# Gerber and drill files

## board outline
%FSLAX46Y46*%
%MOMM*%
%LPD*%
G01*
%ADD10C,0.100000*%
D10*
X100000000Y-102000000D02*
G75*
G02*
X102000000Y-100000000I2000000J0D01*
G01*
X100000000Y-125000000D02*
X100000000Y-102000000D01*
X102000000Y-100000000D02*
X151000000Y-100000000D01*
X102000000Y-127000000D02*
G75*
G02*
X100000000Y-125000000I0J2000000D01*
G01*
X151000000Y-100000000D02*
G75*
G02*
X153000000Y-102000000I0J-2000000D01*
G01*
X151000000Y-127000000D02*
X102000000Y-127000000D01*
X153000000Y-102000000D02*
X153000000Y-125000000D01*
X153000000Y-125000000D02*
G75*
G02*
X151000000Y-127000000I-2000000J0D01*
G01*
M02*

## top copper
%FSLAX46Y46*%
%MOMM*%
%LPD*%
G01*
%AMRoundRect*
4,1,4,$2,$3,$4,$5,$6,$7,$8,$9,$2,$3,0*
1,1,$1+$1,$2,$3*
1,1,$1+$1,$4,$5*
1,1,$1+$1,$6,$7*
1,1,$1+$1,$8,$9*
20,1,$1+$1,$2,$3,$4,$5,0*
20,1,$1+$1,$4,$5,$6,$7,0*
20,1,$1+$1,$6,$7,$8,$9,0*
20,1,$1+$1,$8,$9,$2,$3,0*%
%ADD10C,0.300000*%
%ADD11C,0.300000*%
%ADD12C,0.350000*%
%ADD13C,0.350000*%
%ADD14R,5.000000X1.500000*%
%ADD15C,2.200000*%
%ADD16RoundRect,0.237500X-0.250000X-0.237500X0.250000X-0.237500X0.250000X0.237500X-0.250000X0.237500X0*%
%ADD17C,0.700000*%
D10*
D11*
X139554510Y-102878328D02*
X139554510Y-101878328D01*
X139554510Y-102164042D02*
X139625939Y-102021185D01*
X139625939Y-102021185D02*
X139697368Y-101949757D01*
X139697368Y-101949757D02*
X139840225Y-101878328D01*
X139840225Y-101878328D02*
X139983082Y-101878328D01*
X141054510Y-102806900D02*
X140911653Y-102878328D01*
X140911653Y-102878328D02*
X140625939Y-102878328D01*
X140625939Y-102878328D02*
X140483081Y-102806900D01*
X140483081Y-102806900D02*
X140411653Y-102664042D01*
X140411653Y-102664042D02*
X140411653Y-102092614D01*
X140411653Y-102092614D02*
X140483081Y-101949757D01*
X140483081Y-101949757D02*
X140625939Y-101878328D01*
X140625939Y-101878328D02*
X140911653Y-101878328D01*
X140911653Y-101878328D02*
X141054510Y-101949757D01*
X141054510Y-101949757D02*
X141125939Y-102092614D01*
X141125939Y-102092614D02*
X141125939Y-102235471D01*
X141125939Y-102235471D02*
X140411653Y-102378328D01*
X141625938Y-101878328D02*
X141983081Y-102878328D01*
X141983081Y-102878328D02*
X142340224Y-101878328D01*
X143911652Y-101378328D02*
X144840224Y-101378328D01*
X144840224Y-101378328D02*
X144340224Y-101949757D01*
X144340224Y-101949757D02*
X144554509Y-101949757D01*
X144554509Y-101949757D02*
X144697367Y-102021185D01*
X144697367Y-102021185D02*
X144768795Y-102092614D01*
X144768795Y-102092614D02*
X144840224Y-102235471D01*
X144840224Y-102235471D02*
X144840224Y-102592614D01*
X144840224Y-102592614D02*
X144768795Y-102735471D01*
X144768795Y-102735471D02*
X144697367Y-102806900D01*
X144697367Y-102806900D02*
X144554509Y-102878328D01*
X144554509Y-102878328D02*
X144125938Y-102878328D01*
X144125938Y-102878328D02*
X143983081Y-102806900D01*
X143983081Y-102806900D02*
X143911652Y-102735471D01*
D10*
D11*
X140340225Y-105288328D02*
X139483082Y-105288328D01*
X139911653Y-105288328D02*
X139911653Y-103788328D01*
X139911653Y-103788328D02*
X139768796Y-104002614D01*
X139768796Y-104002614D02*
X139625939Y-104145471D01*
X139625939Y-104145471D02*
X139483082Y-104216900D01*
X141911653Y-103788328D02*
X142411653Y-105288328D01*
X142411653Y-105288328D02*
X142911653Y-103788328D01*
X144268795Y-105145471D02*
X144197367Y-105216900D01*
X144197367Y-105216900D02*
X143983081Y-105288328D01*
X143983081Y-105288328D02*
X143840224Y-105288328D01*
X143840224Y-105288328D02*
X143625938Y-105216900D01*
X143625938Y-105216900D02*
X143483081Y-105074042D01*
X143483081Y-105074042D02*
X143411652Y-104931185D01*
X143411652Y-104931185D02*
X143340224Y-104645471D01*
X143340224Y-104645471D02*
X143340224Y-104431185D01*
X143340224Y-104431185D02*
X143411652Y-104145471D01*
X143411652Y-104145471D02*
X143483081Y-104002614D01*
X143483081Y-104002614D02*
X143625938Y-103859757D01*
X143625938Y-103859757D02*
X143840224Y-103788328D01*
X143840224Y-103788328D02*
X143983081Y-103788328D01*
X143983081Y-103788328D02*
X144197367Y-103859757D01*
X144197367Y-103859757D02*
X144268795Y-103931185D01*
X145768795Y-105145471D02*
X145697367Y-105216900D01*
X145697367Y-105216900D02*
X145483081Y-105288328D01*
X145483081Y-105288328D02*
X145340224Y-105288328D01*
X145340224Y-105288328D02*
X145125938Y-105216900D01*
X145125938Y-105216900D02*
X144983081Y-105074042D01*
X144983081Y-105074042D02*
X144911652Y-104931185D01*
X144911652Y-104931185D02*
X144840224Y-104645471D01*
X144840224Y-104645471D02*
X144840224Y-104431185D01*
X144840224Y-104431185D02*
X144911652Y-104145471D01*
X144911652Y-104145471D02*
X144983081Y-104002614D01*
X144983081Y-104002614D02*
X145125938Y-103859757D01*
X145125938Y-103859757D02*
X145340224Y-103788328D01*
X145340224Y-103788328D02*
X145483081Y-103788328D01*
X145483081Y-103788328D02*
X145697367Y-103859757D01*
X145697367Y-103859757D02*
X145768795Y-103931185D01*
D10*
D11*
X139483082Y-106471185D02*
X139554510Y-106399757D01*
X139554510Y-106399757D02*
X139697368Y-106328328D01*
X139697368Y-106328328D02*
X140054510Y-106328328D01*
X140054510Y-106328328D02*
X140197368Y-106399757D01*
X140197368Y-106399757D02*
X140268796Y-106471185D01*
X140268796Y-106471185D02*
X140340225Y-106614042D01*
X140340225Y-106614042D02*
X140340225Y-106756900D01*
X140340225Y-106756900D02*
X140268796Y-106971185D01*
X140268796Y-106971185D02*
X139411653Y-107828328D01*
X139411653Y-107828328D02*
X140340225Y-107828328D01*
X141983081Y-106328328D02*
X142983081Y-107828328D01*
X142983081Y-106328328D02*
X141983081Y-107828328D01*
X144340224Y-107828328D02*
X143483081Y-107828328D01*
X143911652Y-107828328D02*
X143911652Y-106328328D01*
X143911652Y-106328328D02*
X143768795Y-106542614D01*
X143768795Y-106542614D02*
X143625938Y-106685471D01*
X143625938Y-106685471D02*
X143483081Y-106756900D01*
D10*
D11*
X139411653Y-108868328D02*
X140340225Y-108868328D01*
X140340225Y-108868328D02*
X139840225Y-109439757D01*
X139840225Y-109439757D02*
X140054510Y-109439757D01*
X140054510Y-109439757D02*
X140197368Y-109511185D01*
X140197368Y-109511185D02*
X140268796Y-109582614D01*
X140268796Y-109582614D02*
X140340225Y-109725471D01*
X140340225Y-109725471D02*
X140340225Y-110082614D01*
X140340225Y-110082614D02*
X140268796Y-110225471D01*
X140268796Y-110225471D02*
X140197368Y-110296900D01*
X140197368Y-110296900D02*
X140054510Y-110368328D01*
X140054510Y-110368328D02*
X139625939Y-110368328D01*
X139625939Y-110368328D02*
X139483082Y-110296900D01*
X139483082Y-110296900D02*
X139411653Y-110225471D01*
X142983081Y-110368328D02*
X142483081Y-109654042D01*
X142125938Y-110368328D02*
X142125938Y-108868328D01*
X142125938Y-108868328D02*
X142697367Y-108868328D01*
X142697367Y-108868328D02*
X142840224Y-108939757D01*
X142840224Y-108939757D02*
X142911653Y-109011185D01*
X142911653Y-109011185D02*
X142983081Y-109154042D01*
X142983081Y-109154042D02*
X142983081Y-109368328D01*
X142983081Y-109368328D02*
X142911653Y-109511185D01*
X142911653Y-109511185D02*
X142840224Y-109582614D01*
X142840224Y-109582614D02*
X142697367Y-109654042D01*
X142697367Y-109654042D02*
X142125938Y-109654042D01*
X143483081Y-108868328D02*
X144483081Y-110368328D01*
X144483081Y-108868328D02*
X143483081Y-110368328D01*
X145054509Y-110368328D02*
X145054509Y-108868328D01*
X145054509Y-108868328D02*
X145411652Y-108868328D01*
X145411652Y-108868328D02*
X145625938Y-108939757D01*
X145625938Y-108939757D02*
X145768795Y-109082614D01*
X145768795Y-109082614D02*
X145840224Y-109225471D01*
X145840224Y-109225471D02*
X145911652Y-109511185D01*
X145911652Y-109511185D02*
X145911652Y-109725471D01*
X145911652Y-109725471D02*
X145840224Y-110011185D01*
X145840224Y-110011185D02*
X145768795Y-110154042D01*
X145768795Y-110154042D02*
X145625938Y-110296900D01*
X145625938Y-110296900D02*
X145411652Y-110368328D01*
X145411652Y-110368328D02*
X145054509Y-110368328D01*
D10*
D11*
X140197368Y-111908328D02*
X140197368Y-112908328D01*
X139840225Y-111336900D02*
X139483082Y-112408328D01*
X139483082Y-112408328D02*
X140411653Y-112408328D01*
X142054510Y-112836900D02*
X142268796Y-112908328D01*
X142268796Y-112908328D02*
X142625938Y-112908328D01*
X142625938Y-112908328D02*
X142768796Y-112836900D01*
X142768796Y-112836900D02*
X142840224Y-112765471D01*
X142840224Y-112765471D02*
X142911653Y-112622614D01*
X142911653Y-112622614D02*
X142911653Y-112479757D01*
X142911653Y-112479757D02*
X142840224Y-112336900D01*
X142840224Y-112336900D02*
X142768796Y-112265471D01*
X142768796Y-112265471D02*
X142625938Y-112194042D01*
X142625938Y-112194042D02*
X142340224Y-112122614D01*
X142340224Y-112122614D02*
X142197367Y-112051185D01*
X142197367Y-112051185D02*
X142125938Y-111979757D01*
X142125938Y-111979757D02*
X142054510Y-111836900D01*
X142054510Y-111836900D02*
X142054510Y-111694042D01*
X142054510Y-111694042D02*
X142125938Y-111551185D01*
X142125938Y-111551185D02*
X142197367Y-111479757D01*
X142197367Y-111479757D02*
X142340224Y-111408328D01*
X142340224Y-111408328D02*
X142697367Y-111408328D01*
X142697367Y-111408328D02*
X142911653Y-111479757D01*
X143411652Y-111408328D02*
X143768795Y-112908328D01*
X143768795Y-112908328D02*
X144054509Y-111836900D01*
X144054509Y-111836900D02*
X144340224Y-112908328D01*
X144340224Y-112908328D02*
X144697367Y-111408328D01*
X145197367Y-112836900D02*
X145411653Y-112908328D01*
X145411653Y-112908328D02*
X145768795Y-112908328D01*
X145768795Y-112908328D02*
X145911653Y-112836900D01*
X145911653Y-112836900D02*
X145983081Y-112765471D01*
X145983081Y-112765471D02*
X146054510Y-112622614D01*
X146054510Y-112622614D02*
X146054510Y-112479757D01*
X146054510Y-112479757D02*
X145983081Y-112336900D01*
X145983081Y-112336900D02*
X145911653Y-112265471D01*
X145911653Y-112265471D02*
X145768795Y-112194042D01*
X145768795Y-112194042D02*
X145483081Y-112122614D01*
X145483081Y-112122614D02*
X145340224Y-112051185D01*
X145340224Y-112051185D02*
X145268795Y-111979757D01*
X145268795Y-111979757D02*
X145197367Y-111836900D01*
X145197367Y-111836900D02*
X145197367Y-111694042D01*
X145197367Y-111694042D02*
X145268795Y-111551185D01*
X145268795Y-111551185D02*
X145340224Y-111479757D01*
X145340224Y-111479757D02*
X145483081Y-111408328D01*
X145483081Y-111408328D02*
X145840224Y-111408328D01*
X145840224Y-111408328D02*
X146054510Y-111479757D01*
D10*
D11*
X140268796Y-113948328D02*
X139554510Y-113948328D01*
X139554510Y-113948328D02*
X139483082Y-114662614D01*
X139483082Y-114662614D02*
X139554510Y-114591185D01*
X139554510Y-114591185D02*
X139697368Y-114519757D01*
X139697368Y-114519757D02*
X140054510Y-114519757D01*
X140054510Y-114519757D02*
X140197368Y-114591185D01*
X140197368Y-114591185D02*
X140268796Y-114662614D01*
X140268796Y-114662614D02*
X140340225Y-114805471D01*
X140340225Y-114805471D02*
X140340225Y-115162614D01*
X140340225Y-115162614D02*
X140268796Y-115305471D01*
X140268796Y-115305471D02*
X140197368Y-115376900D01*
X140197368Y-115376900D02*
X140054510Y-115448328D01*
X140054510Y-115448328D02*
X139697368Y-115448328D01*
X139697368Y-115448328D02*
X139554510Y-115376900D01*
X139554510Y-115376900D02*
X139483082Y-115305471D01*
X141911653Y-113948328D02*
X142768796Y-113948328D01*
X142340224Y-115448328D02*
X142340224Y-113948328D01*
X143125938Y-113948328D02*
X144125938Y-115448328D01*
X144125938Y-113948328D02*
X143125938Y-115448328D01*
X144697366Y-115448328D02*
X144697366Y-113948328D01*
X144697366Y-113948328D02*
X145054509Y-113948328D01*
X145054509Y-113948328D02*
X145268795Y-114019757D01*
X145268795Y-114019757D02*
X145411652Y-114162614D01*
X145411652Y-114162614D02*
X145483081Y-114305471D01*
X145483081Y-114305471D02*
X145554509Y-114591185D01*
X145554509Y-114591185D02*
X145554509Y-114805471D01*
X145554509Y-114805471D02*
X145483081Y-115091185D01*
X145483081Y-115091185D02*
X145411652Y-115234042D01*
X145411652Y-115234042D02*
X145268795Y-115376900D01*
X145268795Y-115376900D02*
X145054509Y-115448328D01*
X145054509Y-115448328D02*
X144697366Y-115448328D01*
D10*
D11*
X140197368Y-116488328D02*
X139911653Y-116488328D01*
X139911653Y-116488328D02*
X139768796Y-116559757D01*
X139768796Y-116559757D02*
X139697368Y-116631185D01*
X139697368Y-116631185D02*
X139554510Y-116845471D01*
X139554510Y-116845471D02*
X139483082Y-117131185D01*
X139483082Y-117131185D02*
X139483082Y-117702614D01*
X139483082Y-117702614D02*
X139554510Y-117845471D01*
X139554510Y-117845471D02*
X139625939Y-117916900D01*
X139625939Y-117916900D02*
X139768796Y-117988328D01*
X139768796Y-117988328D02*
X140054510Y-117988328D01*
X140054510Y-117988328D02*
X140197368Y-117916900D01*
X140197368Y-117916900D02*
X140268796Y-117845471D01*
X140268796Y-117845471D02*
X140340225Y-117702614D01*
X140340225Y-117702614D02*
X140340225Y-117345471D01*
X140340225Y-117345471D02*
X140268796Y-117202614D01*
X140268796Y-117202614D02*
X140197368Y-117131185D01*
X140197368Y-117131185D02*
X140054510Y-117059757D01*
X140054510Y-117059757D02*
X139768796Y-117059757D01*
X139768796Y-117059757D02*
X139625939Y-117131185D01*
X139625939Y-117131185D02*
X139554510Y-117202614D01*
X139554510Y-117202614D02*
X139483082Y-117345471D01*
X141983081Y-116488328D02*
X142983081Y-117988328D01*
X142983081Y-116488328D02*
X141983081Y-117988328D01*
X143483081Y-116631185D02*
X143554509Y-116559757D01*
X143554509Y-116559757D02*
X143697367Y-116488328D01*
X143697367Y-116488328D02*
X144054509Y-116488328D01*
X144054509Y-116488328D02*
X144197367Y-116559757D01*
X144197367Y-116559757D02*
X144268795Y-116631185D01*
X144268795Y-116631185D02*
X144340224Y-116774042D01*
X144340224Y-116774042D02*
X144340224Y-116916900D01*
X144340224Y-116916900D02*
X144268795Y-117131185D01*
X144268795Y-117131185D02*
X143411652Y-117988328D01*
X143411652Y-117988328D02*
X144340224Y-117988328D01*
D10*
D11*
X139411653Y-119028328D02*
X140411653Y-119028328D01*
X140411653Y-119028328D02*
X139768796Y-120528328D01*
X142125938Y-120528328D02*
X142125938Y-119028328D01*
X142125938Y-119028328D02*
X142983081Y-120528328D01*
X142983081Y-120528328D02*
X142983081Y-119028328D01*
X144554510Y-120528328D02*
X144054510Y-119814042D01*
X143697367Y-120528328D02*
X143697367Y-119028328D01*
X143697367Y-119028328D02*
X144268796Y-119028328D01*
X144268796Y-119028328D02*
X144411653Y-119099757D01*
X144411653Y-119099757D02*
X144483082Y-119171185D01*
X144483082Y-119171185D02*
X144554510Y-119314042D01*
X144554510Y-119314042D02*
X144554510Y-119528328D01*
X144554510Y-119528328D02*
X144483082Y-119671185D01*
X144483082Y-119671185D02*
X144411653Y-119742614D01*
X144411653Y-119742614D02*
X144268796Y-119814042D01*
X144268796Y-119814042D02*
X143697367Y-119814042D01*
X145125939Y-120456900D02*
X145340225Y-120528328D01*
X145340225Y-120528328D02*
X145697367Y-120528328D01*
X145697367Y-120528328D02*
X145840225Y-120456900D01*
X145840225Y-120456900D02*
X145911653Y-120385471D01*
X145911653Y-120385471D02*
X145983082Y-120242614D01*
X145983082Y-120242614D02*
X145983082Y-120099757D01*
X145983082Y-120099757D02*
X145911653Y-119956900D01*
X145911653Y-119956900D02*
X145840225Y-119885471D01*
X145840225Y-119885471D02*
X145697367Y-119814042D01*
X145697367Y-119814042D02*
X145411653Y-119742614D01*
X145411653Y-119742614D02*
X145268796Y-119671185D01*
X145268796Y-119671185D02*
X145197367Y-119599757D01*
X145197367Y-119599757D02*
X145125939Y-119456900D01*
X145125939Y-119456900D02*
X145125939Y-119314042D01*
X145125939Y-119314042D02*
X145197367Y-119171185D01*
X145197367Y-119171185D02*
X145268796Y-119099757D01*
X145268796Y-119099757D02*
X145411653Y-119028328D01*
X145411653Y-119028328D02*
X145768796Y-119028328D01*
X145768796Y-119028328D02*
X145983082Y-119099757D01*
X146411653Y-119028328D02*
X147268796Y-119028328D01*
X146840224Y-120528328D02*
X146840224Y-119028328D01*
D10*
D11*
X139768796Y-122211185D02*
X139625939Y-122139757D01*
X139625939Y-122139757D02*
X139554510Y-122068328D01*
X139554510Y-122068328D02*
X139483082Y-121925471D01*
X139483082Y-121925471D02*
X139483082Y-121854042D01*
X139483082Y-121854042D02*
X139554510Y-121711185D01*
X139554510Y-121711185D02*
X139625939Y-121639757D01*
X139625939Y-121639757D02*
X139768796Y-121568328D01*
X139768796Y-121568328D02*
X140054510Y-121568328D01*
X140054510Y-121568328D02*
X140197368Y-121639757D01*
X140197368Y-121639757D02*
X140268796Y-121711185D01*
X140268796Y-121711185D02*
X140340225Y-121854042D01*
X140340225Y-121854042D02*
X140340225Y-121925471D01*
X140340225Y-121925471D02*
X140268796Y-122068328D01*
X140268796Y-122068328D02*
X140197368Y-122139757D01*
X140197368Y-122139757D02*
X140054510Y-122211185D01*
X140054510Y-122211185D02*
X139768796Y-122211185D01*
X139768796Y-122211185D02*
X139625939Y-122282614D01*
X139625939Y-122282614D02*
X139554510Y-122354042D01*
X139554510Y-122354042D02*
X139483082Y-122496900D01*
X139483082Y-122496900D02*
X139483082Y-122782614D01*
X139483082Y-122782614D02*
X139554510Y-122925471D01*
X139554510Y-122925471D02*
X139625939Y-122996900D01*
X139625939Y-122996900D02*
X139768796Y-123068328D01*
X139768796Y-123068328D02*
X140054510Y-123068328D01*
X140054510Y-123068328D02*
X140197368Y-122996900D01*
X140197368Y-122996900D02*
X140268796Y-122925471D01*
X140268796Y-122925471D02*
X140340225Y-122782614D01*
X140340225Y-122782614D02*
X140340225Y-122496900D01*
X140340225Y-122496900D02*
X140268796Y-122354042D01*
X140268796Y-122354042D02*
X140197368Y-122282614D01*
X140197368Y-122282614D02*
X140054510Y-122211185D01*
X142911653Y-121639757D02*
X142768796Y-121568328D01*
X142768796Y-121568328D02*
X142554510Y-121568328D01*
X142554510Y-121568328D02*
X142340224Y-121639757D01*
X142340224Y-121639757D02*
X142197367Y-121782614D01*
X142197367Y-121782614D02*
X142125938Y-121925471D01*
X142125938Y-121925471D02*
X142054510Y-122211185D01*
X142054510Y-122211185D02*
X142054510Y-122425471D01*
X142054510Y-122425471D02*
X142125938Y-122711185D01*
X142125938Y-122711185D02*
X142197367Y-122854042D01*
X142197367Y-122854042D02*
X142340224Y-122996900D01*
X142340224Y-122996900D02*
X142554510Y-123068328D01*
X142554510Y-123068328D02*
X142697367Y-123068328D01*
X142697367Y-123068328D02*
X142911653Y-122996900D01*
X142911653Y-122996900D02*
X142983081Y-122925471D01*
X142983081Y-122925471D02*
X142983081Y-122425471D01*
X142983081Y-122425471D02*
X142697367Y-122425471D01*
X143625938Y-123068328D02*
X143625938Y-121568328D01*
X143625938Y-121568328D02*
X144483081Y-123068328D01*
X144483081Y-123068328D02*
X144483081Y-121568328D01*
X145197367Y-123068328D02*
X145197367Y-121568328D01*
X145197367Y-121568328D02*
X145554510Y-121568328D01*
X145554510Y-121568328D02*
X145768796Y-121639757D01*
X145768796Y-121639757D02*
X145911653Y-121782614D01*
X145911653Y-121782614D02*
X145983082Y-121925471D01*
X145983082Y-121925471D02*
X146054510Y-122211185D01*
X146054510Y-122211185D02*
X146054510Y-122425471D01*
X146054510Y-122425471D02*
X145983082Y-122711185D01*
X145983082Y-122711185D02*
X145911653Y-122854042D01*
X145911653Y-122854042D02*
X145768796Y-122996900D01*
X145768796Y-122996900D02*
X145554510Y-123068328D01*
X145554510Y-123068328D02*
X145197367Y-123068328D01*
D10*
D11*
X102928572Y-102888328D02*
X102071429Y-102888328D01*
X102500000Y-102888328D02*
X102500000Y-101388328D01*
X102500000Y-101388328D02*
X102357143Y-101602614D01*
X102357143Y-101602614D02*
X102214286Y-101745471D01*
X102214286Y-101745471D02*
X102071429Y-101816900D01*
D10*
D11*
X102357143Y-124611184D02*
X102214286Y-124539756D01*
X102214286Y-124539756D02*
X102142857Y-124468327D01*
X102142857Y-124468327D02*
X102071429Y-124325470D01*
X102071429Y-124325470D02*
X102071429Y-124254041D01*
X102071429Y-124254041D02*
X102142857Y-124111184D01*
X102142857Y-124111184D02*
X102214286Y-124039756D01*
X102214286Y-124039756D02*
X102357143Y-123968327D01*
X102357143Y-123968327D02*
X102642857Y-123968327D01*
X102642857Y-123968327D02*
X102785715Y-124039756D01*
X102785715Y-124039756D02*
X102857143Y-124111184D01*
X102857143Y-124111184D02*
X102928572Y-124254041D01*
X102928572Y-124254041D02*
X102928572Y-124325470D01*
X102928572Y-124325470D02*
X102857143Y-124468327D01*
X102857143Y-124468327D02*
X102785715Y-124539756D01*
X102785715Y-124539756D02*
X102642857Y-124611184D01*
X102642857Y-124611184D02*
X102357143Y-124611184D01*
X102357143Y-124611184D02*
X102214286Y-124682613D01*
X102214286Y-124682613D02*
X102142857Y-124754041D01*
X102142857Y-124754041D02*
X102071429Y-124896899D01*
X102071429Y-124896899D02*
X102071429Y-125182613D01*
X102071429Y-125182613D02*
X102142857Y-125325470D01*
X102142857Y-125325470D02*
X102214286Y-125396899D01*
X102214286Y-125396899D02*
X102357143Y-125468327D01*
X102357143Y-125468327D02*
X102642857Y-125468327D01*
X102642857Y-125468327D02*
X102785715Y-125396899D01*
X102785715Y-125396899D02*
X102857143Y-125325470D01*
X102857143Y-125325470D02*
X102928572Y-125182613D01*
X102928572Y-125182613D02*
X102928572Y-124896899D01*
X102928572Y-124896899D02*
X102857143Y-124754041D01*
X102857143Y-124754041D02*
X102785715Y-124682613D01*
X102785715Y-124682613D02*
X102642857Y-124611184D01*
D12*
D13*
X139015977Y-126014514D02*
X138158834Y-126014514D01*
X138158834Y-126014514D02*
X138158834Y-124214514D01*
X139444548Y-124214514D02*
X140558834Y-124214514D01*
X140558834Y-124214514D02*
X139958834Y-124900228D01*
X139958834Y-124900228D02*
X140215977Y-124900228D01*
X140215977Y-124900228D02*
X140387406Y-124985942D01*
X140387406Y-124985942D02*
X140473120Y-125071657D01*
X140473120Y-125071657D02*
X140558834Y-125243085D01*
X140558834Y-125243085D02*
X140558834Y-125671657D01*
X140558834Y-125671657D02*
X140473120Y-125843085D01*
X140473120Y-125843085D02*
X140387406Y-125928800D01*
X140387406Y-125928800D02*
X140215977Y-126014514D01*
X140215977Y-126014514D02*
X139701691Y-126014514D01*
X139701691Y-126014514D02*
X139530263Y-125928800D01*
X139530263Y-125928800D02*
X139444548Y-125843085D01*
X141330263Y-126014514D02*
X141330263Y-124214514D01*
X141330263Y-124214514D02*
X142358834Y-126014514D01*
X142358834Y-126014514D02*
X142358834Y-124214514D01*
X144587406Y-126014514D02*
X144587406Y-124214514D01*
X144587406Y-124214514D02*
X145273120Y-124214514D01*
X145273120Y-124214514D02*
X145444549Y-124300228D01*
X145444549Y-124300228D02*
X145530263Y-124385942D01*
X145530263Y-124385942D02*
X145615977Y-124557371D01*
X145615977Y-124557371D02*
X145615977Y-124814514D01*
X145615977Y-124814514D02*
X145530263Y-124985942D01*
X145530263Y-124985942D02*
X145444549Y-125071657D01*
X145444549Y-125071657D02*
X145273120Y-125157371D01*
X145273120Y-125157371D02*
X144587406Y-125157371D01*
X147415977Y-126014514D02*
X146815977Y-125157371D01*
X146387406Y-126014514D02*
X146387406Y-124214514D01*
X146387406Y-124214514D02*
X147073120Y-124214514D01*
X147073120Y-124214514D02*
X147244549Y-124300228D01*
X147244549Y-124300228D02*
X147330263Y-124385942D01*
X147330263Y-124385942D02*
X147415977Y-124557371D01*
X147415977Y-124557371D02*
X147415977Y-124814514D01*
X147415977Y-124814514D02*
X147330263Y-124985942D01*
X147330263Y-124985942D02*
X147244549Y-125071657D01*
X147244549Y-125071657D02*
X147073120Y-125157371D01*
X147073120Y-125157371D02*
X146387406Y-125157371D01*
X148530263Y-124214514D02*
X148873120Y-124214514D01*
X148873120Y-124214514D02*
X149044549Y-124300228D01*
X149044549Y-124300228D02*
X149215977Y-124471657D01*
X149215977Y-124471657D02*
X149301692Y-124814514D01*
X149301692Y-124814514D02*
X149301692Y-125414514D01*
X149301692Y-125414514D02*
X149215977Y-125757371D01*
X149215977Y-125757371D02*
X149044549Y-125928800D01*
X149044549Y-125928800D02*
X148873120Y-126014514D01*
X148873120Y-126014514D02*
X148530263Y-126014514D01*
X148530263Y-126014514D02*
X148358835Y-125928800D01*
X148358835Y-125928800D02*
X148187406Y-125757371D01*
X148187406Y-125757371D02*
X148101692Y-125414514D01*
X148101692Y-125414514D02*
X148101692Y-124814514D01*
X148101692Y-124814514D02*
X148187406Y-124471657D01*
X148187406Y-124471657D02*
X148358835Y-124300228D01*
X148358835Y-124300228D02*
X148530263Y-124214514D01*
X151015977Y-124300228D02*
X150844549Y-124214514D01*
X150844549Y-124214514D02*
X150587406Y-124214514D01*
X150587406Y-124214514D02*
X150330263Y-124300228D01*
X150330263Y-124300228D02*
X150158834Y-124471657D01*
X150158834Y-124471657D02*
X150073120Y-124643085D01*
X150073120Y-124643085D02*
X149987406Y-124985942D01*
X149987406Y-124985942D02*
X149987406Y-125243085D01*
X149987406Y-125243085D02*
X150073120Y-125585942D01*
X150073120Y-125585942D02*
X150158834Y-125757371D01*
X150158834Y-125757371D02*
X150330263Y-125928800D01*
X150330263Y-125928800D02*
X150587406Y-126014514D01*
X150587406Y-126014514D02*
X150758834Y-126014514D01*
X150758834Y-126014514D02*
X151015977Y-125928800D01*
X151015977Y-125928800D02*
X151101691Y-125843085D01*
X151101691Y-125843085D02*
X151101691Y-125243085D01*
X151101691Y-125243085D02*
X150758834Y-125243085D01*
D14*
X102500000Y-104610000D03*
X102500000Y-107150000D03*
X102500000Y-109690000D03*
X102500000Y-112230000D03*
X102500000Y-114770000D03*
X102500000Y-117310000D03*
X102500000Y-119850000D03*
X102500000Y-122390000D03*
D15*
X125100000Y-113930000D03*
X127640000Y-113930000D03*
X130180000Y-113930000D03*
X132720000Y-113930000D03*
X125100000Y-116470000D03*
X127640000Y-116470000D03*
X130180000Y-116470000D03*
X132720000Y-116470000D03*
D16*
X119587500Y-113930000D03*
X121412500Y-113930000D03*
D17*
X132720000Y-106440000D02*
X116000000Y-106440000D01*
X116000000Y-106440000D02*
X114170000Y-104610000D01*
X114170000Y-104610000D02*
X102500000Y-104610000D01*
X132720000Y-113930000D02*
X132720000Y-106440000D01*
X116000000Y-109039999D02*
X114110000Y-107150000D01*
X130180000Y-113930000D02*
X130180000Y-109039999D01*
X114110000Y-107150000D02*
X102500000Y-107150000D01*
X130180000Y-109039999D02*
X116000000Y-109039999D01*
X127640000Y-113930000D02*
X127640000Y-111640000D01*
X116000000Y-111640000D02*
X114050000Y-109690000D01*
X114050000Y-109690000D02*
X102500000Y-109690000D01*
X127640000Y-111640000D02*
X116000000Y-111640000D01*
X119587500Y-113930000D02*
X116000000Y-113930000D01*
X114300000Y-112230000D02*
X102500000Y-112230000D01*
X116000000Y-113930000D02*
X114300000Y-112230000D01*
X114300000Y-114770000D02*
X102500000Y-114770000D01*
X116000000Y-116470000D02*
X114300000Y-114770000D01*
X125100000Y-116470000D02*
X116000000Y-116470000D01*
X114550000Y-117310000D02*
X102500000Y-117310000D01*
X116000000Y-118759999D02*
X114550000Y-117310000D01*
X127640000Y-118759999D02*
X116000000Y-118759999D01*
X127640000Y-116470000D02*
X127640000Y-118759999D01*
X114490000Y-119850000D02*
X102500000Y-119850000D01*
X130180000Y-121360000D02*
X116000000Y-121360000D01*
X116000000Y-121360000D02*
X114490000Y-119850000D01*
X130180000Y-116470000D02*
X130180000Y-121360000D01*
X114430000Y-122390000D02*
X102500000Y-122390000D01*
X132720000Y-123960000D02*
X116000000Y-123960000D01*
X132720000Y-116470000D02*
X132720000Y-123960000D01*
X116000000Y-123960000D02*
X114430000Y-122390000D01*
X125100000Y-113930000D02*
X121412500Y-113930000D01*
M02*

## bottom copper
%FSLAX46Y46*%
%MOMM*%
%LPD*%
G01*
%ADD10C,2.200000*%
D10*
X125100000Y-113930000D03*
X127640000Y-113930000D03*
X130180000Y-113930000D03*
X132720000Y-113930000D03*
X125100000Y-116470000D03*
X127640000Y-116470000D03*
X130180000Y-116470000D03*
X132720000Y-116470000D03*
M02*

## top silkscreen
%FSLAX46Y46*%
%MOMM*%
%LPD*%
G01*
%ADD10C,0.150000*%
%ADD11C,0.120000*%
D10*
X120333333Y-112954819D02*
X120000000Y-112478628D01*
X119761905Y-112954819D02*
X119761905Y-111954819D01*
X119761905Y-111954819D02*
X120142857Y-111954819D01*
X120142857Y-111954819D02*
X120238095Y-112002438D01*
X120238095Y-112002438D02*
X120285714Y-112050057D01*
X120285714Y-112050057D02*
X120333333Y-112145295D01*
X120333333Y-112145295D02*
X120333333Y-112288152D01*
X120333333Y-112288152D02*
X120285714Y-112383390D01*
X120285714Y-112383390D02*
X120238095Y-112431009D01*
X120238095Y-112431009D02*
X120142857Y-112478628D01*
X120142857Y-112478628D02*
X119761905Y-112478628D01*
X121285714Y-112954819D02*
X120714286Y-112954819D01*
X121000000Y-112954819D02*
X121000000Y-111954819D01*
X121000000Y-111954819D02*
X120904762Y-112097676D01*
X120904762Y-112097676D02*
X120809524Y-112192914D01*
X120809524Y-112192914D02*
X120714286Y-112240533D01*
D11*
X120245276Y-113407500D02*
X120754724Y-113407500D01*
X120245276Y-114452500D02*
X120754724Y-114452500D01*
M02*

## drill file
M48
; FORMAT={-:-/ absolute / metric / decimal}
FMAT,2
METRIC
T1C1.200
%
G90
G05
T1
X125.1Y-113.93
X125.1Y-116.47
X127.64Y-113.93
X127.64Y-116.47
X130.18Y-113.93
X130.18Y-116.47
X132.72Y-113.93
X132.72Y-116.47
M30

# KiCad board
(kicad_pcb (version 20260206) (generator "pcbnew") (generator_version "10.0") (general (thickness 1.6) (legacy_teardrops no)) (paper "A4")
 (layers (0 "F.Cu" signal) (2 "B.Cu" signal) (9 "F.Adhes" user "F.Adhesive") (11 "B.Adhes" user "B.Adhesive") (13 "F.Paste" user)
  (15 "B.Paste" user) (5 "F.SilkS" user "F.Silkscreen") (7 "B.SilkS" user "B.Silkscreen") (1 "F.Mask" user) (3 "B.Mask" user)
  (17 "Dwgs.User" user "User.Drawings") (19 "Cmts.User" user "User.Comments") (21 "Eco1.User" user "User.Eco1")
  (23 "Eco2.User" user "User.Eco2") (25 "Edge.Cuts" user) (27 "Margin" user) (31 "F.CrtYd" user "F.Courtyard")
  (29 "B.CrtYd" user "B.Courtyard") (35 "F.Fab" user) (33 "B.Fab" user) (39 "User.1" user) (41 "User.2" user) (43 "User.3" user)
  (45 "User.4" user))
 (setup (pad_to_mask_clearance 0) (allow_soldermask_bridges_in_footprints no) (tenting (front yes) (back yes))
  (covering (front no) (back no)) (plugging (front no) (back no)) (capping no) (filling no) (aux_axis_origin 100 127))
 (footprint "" (layer "F.Cu") (at 102.5 104.61)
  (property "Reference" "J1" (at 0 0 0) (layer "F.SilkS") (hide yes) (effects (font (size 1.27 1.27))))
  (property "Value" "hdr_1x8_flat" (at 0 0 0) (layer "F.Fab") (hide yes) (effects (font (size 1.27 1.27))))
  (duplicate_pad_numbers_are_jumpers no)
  (pad "1" smd rect (at 0 0) (size 5 1.5) (layers "F.Cu" "F.Mask" "F.Paste") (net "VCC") (thermal_bridge_angle 45))
  (pad "2" smd rect (at 0 2.54) (size 5 1.5) (layers "F.Cu" "F.Mask" "F.Paste") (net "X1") (thermal_bridge_angle 45))
  (pad "3" smd rect (at 0 5.08) (size 5 1.5) (layers "F.Cu" "F.Mask" "F.Paste") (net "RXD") (thermal_bridge_angle 45))
  (pad "4" smd rect (at 0 7.62) (size 5 1.5) (layers "F.Cu" "F.Mask" "F.Paste") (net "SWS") (thermal_bridge_angle 45))
  (pad "5" smd rect (at 0 10.16) (size 5 1.5) (layers "F.Cu" "F.Mask" "F.Paste") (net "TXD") (thermal_bridge_angle 45))
  (pad "6" smd rect (at 0 12.7) (size 5 1.5) (layers "F.Cu" "F.Mask" "F.Paste") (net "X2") (thermal_bridge_angle 45))
  (pad "7" smd rect (at 0 15.24) (size 5 1.5) (layers "F.Cu" "F.Mask" "F.Paste") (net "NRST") (thermal_bridge_angle 45))
  (pad "8" smd rect (at 0 17.78) (size 5 1.5) (layers "F.Cu" "F.Mask" "F.Paste") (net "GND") (thermal_bridge_angle 45)))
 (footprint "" (layer "F.Cu") (at 125.1 113.93)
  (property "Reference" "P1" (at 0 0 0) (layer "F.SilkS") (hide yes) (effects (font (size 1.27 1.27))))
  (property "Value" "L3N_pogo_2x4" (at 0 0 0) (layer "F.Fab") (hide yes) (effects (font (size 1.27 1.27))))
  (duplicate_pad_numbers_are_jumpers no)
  (pad "1" thru_hole circle (at 0 0) (size 2.2 2.2) (drill 1.2) (layers "F.Cu") (remove_unused_layers no) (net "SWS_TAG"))
  (pad "2" thru_hole circle (at 2.54 0) (size 2.2 2.2) (drill 1.2) (layers "F.Cu") (remove_unused_layers no) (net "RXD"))
  (pad "3" thru_hole circle (at 5.08 0) (size 2.2 2.2) (drill 1.2) (layers "F.Cu") (remove_unused_layers no) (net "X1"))
  (pad "4" thru_hole circle (at 7.62 0) (size 2.2 2.2) (drill 1.2) (layers "F.Cu") (remove_unused_layers no) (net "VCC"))
  (pad "5" thru_hole circle (at 0 2.54) (size 2.2 2.2) (drill 1.2) (layers "F.Cu") (remove_unused_layers no) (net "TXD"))
  (pad "6" thru_hole circle (at 2.54 2.54) (size 2.2 2.2) (drill 1.2) (layers "F.Cu") (remove_unused_layers no) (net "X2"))
  (pad "7" thru_hole circle (at 5.08 2.54) (size 2.2 2.2) (drill 1.2) (layers "F.Cu") (remove_unused_layers no) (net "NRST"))
  (pad "8" thru_hole circle (at 7.62 2.54) (size 2.2 2.2) (drill 1.2) (layers "F.Cu") (remove_unused_layers no) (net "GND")))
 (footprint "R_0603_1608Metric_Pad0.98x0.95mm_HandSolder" (layer "F.Cu") (at 120.5 113.93)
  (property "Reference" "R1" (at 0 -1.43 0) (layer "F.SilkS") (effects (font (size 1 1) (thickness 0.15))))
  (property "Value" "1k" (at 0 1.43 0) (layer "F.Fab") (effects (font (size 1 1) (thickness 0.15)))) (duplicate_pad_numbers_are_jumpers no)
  (fp_line (start -0.254724 -0.5225) (end 0.254724 -0.5225) (stroke (width 0.12) (type solid)) (layer "F.SilkS"))
  (fp_line (start -0.254724 0.5225) (end 0.254724 0.5225) (stroke (width 0.12) (type solid)) (layer "F.SilkS"))
  (pad "1" smd roundrect (at -0.9125 0) (size 0.975 0.95) (layers "F.Cu" "F.Mask" "F.Paste") (roundrect_rratio 0.25) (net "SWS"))
  (pad "2" smd roundrect (at 0.9125 0) (size 0.975 0.95) (layers "F.Cu" "F.Mask" "F.Paste") (roundrect_rratio 0.25) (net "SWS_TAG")))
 (gr_arc (start 100 102) (mid 100.585786 100.585786) (end 102 100) (stroke (width 0.1) (type default)) (layer "Edge.Cuts"))
 (gr_line (start 100 125) (end 100 102) (stroke (width 0.1) (type default)) (layer "Edge.Cuts"))
 (gr_line (start 102 100) (end 151 100) (stroke (width 0.1) (type default)) (layer "Edge.Cuts"))
 (gr_arc (start 102 127) (mid 100.585786 126.414213) (end 100 125) (stroke (width 0.1) (type default)) (layer "Edge.Cuts"))
 (gr_arc (start 151 100) (mid 152.414213 100.585786) (end 153 102) (stroke (width 0.1) (type default)) (layer "Edge.Cuts"))
 (gr_line (start 151 127) (end 102 127) (stroke (width 0.1) (type default)) (layer "Edge.Cuts"))
 (gr_line (start 153 102) (end 153 125) (stroke (width 0.1) (type default)) (layer "Edge.Cuts"))
 (gr_arc (start 153 125) (mid 152.414213 126.414213) (end 151 127) (stroke (width 0.1) (type default)) (layer "Edge.Cuts"))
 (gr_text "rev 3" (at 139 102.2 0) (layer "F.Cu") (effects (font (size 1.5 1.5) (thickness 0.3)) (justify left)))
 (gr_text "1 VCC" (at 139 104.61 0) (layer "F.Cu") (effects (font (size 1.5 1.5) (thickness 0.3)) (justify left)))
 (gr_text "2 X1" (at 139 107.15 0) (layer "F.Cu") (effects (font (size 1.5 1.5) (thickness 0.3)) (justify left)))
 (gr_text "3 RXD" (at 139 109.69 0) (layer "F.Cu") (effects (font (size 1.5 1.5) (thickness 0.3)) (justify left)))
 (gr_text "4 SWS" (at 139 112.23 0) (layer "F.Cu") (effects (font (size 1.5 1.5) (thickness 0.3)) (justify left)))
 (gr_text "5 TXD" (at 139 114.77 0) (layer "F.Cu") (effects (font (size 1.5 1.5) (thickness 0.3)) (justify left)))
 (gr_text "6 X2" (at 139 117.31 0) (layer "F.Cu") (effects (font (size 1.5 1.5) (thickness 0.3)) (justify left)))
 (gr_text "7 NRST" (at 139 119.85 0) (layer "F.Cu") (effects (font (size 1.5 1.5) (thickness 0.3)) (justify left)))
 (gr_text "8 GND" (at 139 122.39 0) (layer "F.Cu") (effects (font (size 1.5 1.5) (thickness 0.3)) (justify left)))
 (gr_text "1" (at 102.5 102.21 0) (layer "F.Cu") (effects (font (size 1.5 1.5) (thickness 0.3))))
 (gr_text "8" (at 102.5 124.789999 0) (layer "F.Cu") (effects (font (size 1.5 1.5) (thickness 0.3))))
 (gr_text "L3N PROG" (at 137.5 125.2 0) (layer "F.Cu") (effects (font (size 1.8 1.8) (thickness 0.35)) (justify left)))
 (segment (start 132.72 106.44) (end 116 106.44) (width 0.7) (layer "F.Cu") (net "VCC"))
 (segment (start 116 106.44) (end 114.17 104.61) (width 0.7) (layer "F.Cu") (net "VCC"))
 (segment (start 114.17 104.61) (end 102.5 104.61) (width 0.7) (layer "F.Cu") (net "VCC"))
 (segment (start 132.72 113.93) (end 132.72 106.44) (width 0.7) (layer "F.Cu") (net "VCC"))
 (segment (start 116 109.039999) (end 114.11 107.15) (width 0.7) (layer "F.Cu") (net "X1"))
 (segment (start 130.18 113.93) (end 130.18 109.039999) (width 0.7) (layer "F.Cu") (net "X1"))
 (segment (start 114.11 107.15) (end 102.5 107.15) (width 0.7) (layer "F.Cu") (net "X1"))
 (segment (start 130.18 109.039999) (end 116 109.039999) (width 0.7) (layer "F.Cu") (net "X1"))
 (segment (start 127.64 113.93) (end 127.64 111.64) (width 0.7) (layer "F.Cu") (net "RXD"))
 (segment (start 116 111.64) (end 114.05 109.69) (width 0.7) (layer "F.Cu") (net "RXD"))
 (segment (start 114.05 109.69) (end 102.5 109.69) (width 0.7) (layer "F.Cu") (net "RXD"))
 (segment (start 127.64 111.64) (end 116 111.64) (width 0.7) (layer "F.Cu") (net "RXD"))
 (segment (start 119.5875 113.93) (end 116 113.93) (width 0.7) (layer "F.Cu") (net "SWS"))
 (segment (start 114.3 112.23) (end 102.5 112.23) (width 0.7) (layer "F.Cu") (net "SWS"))
 (segment (start 116 113.93) (end 114.3 112.23) (width 0.7) (layer "F.Cu") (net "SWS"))
 (segment (start 114.3 114.77) (end 102.5 114.77) (width 0.7) (layer "F.Cu") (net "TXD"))
 (segment (start 116 116.47) (end 114.3 114.77) (width 0.7) (layer "F.Cu") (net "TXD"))
 (segment (start 125.1 116.47) (end 116 116.47) (width 0.7) (layer "F.Cu") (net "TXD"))
 (segment (start 114.55 117.31) (end 102.5 117.31) (width 0.7) (layer "F.Cu") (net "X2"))
 (segment (start 116 118.759999) (end 114.55 117.31) (width 0.7) (layer "F.Cu") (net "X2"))
 (segment (start 127.64 118.759999) (end 116 118.759999) (width 0.7) (layer "F.Cu") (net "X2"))
 (segment (start 127.64 116.47) (end 127.64 118.759999) (width 0.7) (layer "F.Cu") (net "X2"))
 (segment (start 114.49 119.85) (end 102.5 119.85) (width 0.7) (layer "F.Cu") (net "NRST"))
 (segment (start 130.18 121.36) (end 116 121.36) (width 0.7) (layer "F.Cu") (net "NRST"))
 (segment (start 116 121.36) (end 114.49 119.85) (width 0.7) (layer "F.Cu") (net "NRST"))
 (segment (start 130.18 116.47) (end 130.18 121.36) (width 0.7) (layer "F.Cu") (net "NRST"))
 (segment (start 114.43 122.39) (end 102.5 122.39) (width 0.7) (layer "F.Cu") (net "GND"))
 (segment (start 132.72 123.96) (end 116 123.96) (width 0.7) (layer "F.Cu") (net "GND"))
 (segment (start 132.72 116.47) (end 132.72 123.96) (width 0.7) (layer "F.Cu") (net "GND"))
 (segment (start 116 123.96) (end 114.43 122.39) (width 0.7) (layer "F.Cu") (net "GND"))
 (segment (start 125.1 113.93) (end 121.4125 113.93) (width 0.7) (layer "F.Cu") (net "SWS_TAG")))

